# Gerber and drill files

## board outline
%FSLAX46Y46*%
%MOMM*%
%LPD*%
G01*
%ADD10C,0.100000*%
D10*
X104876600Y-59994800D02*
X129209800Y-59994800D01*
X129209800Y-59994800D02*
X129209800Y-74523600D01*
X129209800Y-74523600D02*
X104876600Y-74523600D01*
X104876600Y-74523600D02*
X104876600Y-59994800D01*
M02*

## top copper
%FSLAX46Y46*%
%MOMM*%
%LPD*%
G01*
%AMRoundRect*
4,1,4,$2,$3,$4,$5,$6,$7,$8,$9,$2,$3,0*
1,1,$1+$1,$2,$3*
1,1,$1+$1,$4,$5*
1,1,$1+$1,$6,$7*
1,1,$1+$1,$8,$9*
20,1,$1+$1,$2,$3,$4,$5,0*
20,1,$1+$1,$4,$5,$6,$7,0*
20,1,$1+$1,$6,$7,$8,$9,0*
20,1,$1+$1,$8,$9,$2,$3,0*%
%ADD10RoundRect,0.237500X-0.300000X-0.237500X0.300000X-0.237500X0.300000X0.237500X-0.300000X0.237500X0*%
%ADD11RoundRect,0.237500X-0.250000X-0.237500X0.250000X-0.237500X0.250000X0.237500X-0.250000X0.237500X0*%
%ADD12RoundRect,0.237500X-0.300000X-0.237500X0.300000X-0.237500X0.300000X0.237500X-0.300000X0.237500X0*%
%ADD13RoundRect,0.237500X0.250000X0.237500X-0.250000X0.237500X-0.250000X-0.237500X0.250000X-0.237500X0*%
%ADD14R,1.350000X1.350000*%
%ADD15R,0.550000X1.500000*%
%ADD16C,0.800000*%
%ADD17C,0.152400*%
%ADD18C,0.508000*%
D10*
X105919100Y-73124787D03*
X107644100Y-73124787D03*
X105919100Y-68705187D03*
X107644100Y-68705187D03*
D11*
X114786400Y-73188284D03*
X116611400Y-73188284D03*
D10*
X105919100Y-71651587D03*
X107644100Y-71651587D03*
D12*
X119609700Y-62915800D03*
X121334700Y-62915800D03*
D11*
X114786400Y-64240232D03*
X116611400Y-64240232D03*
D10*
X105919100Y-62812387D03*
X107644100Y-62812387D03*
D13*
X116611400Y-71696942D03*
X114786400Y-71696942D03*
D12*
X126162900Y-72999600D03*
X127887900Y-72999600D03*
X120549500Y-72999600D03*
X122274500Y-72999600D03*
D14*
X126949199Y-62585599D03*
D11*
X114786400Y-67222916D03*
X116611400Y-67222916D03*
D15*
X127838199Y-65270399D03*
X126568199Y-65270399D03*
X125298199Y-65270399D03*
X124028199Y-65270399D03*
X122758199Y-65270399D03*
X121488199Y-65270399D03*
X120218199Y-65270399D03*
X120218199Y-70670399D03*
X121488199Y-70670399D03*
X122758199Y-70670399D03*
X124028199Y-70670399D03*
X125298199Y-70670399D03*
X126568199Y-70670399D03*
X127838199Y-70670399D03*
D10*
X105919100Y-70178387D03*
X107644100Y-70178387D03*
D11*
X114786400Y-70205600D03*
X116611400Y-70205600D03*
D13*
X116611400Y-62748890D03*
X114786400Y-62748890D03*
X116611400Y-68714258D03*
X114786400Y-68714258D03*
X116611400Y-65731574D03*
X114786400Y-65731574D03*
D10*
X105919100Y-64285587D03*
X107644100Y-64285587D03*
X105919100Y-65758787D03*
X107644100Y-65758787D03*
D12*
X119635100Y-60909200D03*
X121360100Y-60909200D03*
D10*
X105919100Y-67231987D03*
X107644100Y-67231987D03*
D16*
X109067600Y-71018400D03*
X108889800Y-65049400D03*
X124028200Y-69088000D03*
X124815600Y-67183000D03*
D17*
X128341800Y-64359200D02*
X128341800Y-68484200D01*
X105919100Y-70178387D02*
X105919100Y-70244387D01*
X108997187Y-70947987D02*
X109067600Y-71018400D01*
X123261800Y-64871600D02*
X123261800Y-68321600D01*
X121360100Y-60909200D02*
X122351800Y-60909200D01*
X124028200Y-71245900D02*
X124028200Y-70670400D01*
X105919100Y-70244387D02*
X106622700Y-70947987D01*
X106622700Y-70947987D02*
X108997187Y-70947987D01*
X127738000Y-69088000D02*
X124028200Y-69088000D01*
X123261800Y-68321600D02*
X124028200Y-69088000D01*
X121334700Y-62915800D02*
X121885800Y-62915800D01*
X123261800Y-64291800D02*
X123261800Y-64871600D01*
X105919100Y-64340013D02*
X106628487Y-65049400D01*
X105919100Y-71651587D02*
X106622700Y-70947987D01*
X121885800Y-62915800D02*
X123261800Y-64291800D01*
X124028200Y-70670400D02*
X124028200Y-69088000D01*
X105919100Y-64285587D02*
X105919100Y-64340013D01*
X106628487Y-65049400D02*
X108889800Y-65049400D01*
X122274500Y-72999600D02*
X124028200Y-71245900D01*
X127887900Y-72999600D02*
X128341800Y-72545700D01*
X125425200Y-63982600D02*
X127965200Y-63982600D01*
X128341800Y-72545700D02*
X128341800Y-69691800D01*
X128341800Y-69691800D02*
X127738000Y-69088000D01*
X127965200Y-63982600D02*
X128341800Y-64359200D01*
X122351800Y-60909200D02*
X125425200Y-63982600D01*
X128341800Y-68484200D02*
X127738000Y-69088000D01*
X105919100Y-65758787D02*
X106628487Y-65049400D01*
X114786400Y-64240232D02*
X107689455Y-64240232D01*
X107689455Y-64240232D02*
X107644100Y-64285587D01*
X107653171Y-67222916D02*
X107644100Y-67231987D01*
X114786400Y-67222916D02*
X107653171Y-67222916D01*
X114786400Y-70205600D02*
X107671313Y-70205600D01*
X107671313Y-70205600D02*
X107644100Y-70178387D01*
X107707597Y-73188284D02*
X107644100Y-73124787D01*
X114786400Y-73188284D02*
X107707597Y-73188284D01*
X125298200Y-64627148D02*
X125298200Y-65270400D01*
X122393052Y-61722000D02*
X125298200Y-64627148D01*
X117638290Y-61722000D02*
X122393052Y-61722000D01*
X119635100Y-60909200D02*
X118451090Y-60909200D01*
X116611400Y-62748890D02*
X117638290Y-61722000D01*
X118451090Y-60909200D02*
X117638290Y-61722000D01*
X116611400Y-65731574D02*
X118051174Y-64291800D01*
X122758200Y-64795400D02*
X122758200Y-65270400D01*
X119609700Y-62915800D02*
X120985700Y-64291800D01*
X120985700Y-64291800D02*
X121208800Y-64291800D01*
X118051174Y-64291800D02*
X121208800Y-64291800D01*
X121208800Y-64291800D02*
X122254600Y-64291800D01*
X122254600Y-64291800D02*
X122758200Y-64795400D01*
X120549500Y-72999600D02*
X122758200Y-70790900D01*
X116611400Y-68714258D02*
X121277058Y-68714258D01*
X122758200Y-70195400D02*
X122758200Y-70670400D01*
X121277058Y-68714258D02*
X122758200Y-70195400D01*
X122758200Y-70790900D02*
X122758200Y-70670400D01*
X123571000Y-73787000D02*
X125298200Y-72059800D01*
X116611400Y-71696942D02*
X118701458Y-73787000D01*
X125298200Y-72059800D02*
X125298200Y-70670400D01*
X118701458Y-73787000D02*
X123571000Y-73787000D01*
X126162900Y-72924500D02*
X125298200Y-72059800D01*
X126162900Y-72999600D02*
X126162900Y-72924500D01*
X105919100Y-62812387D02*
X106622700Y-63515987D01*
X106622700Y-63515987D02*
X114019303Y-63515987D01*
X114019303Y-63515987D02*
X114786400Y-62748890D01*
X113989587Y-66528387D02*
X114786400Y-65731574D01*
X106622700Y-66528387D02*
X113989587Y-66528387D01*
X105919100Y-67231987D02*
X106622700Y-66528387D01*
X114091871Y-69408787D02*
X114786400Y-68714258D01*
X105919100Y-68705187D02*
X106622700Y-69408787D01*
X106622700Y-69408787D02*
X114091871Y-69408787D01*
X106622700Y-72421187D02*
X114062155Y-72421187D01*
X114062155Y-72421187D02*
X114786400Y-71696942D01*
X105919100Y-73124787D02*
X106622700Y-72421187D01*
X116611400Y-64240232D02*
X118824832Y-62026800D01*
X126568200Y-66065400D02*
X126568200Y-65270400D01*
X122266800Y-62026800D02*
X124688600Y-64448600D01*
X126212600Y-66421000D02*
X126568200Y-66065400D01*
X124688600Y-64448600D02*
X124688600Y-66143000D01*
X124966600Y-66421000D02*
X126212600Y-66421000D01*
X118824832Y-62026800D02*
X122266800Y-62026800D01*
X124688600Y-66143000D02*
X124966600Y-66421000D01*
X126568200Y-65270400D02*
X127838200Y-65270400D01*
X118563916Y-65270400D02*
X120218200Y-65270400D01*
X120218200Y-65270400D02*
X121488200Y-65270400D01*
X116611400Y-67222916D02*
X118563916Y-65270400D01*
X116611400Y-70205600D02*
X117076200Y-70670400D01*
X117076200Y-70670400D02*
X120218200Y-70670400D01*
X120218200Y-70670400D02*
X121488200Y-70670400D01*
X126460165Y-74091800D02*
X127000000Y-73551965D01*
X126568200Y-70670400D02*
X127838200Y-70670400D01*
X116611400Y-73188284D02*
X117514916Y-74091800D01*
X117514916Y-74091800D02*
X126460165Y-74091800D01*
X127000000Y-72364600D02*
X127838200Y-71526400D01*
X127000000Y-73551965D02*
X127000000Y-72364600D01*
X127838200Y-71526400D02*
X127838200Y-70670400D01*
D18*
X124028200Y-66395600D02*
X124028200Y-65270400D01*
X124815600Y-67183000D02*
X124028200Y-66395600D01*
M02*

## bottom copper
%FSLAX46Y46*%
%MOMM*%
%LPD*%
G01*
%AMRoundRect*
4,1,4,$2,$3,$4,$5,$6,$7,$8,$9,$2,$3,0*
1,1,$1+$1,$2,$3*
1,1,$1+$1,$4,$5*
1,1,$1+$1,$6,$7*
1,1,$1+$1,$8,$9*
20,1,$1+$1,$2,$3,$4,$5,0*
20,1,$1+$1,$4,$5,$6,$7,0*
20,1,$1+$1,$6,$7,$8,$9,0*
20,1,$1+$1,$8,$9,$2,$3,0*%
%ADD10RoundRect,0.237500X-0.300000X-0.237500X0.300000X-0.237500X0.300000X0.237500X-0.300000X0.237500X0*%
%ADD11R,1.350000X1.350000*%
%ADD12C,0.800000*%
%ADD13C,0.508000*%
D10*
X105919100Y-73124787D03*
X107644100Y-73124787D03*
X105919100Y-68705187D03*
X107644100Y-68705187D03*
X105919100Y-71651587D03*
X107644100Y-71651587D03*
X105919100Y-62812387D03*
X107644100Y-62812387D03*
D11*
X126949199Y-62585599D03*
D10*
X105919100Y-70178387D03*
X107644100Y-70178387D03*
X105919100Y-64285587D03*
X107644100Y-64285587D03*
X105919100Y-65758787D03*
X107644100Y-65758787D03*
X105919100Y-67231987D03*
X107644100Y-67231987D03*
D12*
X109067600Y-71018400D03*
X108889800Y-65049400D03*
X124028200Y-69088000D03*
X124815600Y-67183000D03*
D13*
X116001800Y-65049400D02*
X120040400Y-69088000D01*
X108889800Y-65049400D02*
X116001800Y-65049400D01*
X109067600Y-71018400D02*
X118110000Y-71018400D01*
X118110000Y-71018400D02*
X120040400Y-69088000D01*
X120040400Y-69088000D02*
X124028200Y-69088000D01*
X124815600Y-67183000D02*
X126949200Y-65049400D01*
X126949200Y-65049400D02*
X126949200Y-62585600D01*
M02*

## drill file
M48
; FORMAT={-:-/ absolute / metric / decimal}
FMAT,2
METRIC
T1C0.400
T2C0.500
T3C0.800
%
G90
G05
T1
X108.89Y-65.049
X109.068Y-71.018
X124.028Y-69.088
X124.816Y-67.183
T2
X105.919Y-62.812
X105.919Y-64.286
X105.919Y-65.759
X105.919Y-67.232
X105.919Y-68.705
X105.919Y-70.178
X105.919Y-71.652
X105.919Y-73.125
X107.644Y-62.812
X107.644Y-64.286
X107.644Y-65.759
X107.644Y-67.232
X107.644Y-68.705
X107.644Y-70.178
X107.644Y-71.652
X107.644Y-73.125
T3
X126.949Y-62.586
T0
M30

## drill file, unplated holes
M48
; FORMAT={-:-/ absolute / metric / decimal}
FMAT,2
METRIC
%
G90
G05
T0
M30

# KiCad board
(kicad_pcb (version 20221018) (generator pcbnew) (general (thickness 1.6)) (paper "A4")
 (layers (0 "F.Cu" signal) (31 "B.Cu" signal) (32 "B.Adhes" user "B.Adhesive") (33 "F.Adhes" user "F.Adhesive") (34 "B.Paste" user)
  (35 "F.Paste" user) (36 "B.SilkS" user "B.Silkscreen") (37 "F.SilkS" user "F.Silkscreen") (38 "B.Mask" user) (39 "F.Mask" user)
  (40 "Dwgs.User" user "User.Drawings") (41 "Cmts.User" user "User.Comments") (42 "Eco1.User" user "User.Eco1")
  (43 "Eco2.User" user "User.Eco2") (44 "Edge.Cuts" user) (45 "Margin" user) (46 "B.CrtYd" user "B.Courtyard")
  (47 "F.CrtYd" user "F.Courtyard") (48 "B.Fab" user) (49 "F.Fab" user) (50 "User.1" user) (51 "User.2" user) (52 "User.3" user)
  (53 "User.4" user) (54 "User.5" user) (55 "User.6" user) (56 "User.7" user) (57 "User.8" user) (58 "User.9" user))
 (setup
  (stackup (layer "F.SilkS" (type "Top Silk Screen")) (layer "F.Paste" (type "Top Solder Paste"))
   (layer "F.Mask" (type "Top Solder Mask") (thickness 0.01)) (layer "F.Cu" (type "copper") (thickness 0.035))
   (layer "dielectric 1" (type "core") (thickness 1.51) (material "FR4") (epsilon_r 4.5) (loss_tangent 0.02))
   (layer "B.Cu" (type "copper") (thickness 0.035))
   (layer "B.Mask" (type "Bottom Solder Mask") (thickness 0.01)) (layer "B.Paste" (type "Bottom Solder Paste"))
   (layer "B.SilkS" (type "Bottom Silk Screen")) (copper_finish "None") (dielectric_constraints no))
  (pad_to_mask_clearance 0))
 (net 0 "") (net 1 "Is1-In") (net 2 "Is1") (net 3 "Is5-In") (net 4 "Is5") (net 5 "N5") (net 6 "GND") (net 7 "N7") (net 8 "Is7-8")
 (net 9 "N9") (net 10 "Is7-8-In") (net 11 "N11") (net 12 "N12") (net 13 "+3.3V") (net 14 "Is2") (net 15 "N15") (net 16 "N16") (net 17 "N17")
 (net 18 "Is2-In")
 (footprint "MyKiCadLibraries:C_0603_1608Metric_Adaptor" (layer "F.Cu") (at 106.7816 73.124787)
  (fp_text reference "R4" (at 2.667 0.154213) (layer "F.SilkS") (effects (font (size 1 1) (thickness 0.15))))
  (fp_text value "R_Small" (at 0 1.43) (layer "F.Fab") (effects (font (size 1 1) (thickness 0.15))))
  (pad "1" thru_hole roundrect (at -0.8625 0) (size 1.075 0.95) (drill 0.5) (layers "*.Cu" "*.Mask") (roundrect_rratio 0.25)
   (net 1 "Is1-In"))
  (pad "2" thru_hole roundrect (at 0.8625 0) (size 1.075 0.95) (drill 0.5) (layers "*.Cu" "*.Mask") (roundrect_rratio 0.25) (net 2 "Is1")))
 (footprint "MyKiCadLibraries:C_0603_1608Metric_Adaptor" (layer "F.Cu") (at 106.7816 68.705187)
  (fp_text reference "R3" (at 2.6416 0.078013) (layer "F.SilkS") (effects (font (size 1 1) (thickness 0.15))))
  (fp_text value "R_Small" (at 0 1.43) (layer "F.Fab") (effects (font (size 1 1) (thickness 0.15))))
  (pad "1" thru_hole roundrect (at -0.8625 0) (size 1.075 0.95) (drill 0.5) (layers "*.Cu" "*.Mask") (roundrect_rratio 0.25)
   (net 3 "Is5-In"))
  (pad "2" thru_hole roundrect (at 0.8625 0) (size 1.075 0.95) (drill 0.5) (layers "*.Cu" "*.Mask") (roundrect_rratio 0.25) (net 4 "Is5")))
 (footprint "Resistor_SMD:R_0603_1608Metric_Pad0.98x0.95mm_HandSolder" (layer "F.Cu") (at 115.6989 73.188284)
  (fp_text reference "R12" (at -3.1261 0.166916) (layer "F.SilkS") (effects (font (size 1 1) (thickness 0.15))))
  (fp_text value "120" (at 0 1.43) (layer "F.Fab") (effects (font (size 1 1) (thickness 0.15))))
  (pad "1" smd roundrect (at -0.9125 0) (size 0.975 0.95) (layers "F.Cu" "F.Paste" "F.Mask") (roundrect_rratio 0.25) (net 2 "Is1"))
  (pad "2" smd roundrect (at 0.9125 0) (size 0.975 0.95) (layers "F.Cu" "F.Paste" "F.Mask") (roundrect_rratio 0.25) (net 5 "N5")))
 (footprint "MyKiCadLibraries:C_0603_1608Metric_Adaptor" (layer "F.Cu") (at 106.7816 71.651587)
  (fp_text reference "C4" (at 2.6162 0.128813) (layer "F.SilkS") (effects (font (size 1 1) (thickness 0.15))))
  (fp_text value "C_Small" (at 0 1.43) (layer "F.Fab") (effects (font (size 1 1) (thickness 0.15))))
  (pad "1" thru_hole roundrect (at -0.8625 0) (size 1.075 0.95) (drill 0.5) (layers "*.Cu" "*.Mask") (roundrect_rratio 0.25) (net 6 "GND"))
  (pad "2" thru_hole roundrect (at 0.8625 0) (size 1.075 0.95) (drill 0.5) (layers "*.Cu" "*.Mask") (roundrect_rratio 0.25) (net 2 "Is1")))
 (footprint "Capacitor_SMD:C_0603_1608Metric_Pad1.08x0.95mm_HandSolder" (layer "F.Cu") (at 120.4722 62.9158)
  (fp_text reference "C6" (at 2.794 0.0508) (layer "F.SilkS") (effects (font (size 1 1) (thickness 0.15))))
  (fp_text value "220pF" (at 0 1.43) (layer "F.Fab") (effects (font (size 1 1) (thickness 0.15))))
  (pad "1" smd roundrect (at -0.8625 0) (size 1.075 0.95) (layers "F.Cu" "F.Paste" "F.Mask") (roundrect_rratio 0.25) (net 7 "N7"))
  (pad "2" smd roundrect (at 0.8625 0) (size 1.075 0.95) (layers "F.Cu" "F.Paste" "F.Mask") (roundrect_rratio 0.25) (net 6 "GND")))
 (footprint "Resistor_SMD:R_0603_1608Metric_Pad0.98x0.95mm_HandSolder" (layer "F.Cu") (at 115.6989 64.240232)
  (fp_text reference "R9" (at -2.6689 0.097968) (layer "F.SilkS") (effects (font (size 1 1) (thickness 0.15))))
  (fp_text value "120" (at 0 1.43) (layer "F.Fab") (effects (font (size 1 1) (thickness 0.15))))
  (pad "1" smd roundrect (at -0.9125 0) (size 0.975 0.95) (layers "F.Cu" "F.Paste" "F.Mask") (roundrect_rratio 0.25) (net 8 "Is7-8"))
  (pad "2" smd roundrect (at 0.9125 0) (size 0.975 0.95) (layers "F.Cu" "F.Paste" "F.Mask") (roundrect_rratio 0.25) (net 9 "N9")))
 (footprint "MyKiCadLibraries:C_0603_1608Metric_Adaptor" (layer "F.Cu") (at 106.7816 62.812387)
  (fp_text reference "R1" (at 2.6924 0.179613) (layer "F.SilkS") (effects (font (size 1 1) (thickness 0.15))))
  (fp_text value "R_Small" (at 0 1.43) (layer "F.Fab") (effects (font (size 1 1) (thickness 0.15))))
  (pad "1" thru_hole roundrect (at -0.8625 0) (size 1.075 0.95) (drill 0.5) (layers "*.Cu" "*.Mask") (roundrect_rratio 0.25)
   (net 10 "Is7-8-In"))
  (pad "2" thru_hole roundrect (at 0.8625 0) (size 1.075 0.95) (drill 0.5) (layers "*.Cu" "*.Mask") (roundrect_rratio 0.25) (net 8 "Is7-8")))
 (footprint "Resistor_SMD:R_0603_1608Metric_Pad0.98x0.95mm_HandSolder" (layer "F.Cu") (at 115.6989 71.696942 180)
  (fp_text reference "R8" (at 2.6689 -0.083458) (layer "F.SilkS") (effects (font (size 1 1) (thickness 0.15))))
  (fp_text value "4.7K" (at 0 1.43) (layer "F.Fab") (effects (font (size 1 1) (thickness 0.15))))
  (pad "1" smd roundrect (at -0.9125 0 180) (size 0.975 0.95) (layers "F.Cu" "F.Paste" "F.Mask") (roundrect_rratio 0.25) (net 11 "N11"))
  (pad "2" smd roundrect (at 0.9125 0 180) (size 0.975 0.95) (layers "F.Cu" "F.Paste" "F.Mask") (roundrect_rratio 0.25) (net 1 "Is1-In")))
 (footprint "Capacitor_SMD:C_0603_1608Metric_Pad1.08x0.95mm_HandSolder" (layer "F.Cu") (at 127.0254 72.9996)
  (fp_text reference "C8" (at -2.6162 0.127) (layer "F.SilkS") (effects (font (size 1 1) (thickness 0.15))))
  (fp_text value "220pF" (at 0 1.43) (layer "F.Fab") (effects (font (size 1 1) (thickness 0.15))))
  (pad "1" smd roundrect (at -0.8625 0) (size 1.075 0.95) (layers "F.Cu" "F.Paste" "F.Mask") (roundrect_rratio 0.25) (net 11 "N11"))
  (pad "2" smd roundrect (at 0.8625 0) (size 1.075 0.95) (layers "F.Cu" "F.Paste" "F.Mask") (roundrect_rratio 0.25) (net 6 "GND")))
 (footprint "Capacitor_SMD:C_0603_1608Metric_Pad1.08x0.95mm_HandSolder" (layer "F.Cu") (at 121.412 72.9996)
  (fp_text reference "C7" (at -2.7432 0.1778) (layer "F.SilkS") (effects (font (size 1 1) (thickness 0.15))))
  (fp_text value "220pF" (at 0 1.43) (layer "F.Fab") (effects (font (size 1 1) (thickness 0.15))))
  (pad "1" smd roundrect (at -0.8625 0) (size 1.075 0.95) (layers "F.Cu" "F.Paste" "F.Mask") (roundrect_rratio 0.25) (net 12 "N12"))
  (pad "2" smd roundrect (at 0.8625 0) (size 1.075 0.95) (layers "F.Cu" "F.Paste" "F.Mask") (roundrect_rratio 0.25) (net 6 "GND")))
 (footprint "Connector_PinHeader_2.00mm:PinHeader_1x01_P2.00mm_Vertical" (layer "F.Cu") (at 126.9492 62.5856)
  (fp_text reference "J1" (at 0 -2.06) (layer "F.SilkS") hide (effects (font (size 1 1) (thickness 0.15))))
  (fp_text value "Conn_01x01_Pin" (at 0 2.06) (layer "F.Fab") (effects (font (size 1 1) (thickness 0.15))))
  (pad "1" thru_hole rect (at 0 0) (size 1.35 1.35) (drill 0.8) (layers "*.Cu" "*.Mask") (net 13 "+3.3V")))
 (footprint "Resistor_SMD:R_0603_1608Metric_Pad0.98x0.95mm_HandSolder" (layer "F.Cu") (at 115.6989 67.222916)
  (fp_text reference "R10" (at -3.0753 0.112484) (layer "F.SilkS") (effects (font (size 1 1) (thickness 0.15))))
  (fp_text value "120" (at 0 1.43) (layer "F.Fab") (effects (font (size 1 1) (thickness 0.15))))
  (pad "1" smd roundrect (at -0.9125 0) (size 0.975 0.95) (layers "F.Cu" "F.Paste" "F.Mask") (roundrect_rratio 0.25) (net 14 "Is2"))
  (pad "2" smd roundrect (at 0.9125 0) (size 0.975 0.95) (layers "F.Cu" "F.Paste" "F.Mask") (roundrect_rratio 0.25) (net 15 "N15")))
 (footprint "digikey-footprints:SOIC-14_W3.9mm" (layer "F.Cu") (at 124.0282 67.9704 180)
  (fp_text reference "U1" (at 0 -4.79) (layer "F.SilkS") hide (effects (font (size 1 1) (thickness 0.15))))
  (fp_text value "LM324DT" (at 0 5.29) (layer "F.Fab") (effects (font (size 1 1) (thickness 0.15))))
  (pad "1" smd rect (at -3.81 2.7 180) (size 0.55 1.5) (layers "F.Cu" "F.Paste" "F.Mask") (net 9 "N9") (solder_mask_margin 0.07))
  (pad "2" smd rect (at -2.54 2.7 180) (size 0.55 1.5) (layers "F.Cu" "F.Paste" "F.Mask") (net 9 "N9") (solder_mask_margin 0.07))
  (pad "3" smd rect (at -1.27 2.7 180) (size 0.55 1.5) (layers "F.Cu" "F.Paste" "F.Mask") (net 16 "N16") (solder_mask_margin 0.07))
  (pad "4" smd rect (at 0 2.7 180) (size 0.55 1.5) (layers "F.Cu" "F.Paste" "F.Mask") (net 13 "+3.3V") (solder_mask_margin 0.07))
  (pad "5" smd rect (at 1.27 2.7 180) (size 0.55 1.5) (layers "F.Cu" "F.Paste" "F.Mask") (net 7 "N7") (solder_mask_margin 0.07))
  (pad "6" smd rect (at 2.54 2.7 180) (size 0.55 1.5) (layers "F.Cu" "F.Paste" "F.Mask") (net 15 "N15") (solder_mask_margin 0.07))
  (pad "7" smd rect (at 3.81 2.7 180) (size 0.55 1.5) (layers "F.Cu" "F.Paste" "F.Mask") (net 15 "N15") (solder_mask_margin 0.07))
  (pad "8" smd rect (at 3.81 -2.7 180) (size 0.55 1.5) (layers "F.Cu" "F.Paste" "F.Mask") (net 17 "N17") (solder_mask_margin 0.07))
  (pad "9" smd rect (at 2.54 -2.7 180) (size 0.55 1.5) (layers "F.Cu" "F.Paste" "F.Mask") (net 17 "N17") (solder_mask_margin 0.07))
  (pad "10" smd rect (at 1.27 -2.7 180) (size 0.55 1.5) (layers "F.Cu" "F.Paste" "F.Mask") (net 12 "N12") (solder_mask_margin 0.07))
  (pad "11" smd rect (at 0 -2.7 180) (size 0.55 1.5) (layers "F.Cu" "F.Paste" "F.Mask") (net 6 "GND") (solder_mask_margin 0.07))
  (pad "12" smd rect (at -1.27 -2.7 180) (size 0.55 1.5) (layers "F.Cu" "F.Paste" "F.Mask") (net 11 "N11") (solder_mask_margin 0.07))
  (pad "13" smd rect (at -2.54 -2.7 180) (size 0.55 1.5) (layers "F.Cu" "F.Paste" "F.Mask") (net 5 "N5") (solder_mask_margin 0.07))
  (pad "14" smd rect (at -3.81 -2.7 180) (size 0.55 1.5) (layers "F.Cu" "F.Paste" "F.Mask") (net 5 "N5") (solder_mask_margin 0.07)))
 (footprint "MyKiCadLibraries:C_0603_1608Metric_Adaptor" (layer "F.Cu") (at 106.7816 70.178387)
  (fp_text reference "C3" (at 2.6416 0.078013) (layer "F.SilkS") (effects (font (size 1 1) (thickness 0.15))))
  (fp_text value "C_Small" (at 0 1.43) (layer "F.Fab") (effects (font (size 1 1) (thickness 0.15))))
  (pad "1" thru_hole roundrect (at -0.8625 0) (size 1.075 0.95) (drill 0.5) (layers "*.Cu" "*.Mask") (roundrect_rratio 0.25) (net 6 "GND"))
  (pad "2" thru_hole roundrect (at 0.8625 0) (size 1.075 0.95) (drill 0.5) (layers "*.Cu" "*.Mask") (roundrect_rratio 0.25) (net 4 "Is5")))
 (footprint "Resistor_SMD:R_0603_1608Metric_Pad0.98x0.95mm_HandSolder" (layer "F.Cu") (at 115.6989 70.2056)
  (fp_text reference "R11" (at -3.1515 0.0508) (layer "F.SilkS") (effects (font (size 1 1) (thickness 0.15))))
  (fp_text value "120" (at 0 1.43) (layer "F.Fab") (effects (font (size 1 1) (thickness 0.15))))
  (pad "1" smd roundrect (at -0.9125 0) (size 0.975 0.95) (layers "F.Cu" "F.Paste" "F.Mask") (roundrect_rratio 0.25) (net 4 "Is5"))
  (pad "2" smd roundrect (at 0.9125 0) (size 0.975 0.95) (layers "F.Cu" "F.Paste" "F.Mask") (roundrect_rratio 0.25) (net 17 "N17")))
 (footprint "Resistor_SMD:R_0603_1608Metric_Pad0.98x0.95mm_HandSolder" (layer "F.Cu") (at 115.6989 62.74889 180)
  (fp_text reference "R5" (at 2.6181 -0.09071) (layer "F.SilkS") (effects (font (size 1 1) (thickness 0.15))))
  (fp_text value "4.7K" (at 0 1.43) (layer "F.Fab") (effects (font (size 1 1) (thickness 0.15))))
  (pad "1" smd roundrect (at -0.9125 0 180) (size 0.975 0.95) (layers "F.Cu" "F.Paste" "F.Mask") (roundrect_rratio 0.25) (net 16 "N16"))
  (pad "2" smd roundrect (at 0.9125 0 180) (size 0.975 0.95) (layers "F.Cu" "F.Paste" "F.Mask") (roundrect_rratio 0.25) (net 10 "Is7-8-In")))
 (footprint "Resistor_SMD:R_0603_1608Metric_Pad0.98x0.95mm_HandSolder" (layer "F.Cu") (at 115.6989 68.714258 180)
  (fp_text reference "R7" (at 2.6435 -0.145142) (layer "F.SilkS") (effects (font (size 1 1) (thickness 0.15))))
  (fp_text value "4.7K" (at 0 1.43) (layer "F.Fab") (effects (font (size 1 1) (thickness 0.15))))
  (pad "1" smd roundrect (at -0.9125 0 180) (size 0.975 0.95) (layers "F.Cu" "F.Paste" "F.Mask") (roundrect_rratio 0.25) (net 12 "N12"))
  (pad "2" smd roundrect (at 0.9125 0 180) (size 0.975 0.95) (layers "F.Cu" "F.Paste" "F.Mask") (roundrect_rratio 0.25) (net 3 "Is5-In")))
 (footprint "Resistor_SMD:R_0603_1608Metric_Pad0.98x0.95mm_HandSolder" (layer "F.Cu") (at 115.6989 65.731574 180)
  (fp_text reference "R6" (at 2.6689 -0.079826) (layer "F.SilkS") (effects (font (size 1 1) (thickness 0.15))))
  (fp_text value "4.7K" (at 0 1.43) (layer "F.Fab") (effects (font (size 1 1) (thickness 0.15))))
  (pad "1" smd roundrect (at -0.9125 0 180) (size 0.975 0.95) (layers "F.Cu" "F.Paste" "F.Mask") (roundrect_rratio 0.25) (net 7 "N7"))
  (pad "2" smd roundrect (at 0.9125 0 180) (size 0.975 0.95) (layers "F.Cu" "F.Paste" "F.Mask") (roundrect_rratio 0.25) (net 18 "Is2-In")))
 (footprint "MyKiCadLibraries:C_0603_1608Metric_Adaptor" (layer "F.Cu") (at 106.7816 64.285587)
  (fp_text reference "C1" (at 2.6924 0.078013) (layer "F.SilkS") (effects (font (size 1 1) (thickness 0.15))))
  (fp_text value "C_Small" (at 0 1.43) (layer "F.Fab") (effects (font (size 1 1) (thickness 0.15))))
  (pad "1" thru_hole roundrect (at -0.8625 0) (size 1.075 0.95) (drill 0.5) (layers "*.Cu" "*.Mask") (roundrect_rratio 0.25) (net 6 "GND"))
  (pad "2" thru_hole roundrect (at 0.8625 0) (size 1.075 0.95) (drill 0.5) (layers "*.Cu" "*.Mask") (roundrect_rratio 0.25) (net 8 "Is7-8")))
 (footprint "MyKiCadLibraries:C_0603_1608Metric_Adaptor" (layer "F.Cu") (at 106.7816 65.758787)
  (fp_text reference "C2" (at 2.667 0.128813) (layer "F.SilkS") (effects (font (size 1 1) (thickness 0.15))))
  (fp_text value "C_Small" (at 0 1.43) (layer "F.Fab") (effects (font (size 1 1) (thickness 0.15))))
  (pad "1" thru_hole roundrect (at -0.8625 0) (size 1.075 0.95) (drill 0.5) (layers "*.Cu" "*.Mask") (roundrect_rratio 0.25) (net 6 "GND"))
  (pad "2" thru_hole roundrect (at 0.8625 0) (size 1.075 0.95) (drill 0.5) (layers "*.Cu" "*.Mask") (roundrect_rratio 0.25) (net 14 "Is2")))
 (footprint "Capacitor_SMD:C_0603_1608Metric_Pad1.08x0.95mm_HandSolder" (layer "F.Cu") (at 120.4976 60.9092)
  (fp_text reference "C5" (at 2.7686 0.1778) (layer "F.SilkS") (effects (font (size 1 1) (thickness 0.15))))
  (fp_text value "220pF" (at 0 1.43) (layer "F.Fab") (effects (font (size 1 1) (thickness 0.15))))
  (pad "1" smd roundrect (at -0.8625 0) (size 1.075 0.95) (layers "F.Cu" "F.Paste" "F.Mask") (roundrect_rratio 0.25) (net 16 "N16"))
  (pad "2" smd roundrect (at 0.8625 0) (size 1.075 0.95) (layers "F.Cu" "F.Paste" "F.Mask") (roundrect_rratio 0.25) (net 6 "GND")))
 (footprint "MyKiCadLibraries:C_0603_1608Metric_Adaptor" (layer "F.Cu") (at 106.7816 67.231987)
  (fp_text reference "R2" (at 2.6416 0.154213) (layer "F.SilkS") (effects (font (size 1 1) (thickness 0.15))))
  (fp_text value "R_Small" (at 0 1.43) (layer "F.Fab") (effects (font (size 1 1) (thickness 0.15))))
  (pad "1" thru_hole roundrect (at -0.8625 0) (size 1.075 0.95) (drill 0.5) (layers "*.Cu" "*.Mask") (roundrect_rratio 0.25)
   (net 18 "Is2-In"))
  (pad "2" thru_hole roundrect (at 0.8625 0) (size 1.075 0.95) (drill 0.5) (layers "*.Cu" "*.Mask") (roundrect_rratio 0.25) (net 14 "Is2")))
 (gr_rect (start 104.8766 59.9948) (end 129.2098 74.5236) (stroke (width 0.1) (type default)) (fill none) (layer "Edge.Cuts"))
 (segment (start 128.3418 64.3592) (end 128.3418 68.4842) (width 0.1524) (layer "F.Cu") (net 6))
 (segment (start 105.9191 70.178387) (end 105.9191 70.244387) (width 0.1524) (layer "F.Cu") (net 6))
 (segment (start 108.997187 70.947987) (end 109.0676 71.0184) (width 0.1524) (layer "F.Cu") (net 6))
 (segment (start 123.2618 64.8716) (end 123.2618 68.3216) (width 0.1524) (layer "F.Cu") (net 6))
 (segment (start 121.3601 60.9092) (end 122.3518 60.9092) (width 0.1524) (layer "F.Cu") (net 6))
 (segment (start 124.0282 71.2459) (end 124.0282 70.6704) (width 0.1524) (layer "F.Cu") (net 6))
 (segment (start 105.9191 70.244387) (end 106.6227 70.947987) (width 0.1524) (layer "F.Cu") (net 6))
 (segment (start 106.6227 70.947987) (end 108.997187 70.947987) (width 0.1524) (layer "F.Cu") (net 6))
 (segment (start 127.738 69.088) (end 124.0282 69.088) (width 0.1524) (layer "F.Cu") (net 6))
 (segment (start 123.2618 68.3216) (end 124.0282 69.088) (width 0.1524) (layer "F.Cu") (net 6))
 (segment (start 121.3347 62.9158) (end 121.8858 62.9158) (width 0.1524) (layer "F.Cu") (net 6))
 (segment (start 123.2618 64.2918) (end 123.2618 64.8716) (width 0.1524) (layer "F.Cu") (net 6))
 (segment (start 105.9191 64.340013) (end 106.628487 65.0494) (width 0.1524) (layer "F.Cu") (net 6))
 (segment (start 105.9191 71.651587) (end 106.6227 70.947987) (width 0.1524) (layer "F.Cu") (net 6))
 (segment (start 121.8858 62.9158) (end 123.2618 64.2918) (width 0.1524) (layer "F.Cu") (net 6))
 (segment (start 124.0282 70.6704) (end 124.0282 69.088) (width 0.1524) (layer "F.Cu") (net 6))
 (segment (start 105.9191 64.285587) (end 105.9191 64.340013) (width 0.1524) (layer "F.Cu") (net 6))
 (segment (start 106.628487 65.0494) (end 108.8898 65.0494) (width 0.1524) (layer "F.Cu") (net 6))
 (segment (start 122.2745 72.9996) (end 124.0282 71.2459) (width 0.1524) (layer "F.Cu") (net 6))
 (segment (start 127.8879 72.9996) (end 128.3418 72.5457) (width 0.1524) (layer "F.Cu") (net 6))
 (segment (start 125.4252 63.9826) (end 127.9652 63.9826) (width 0.1524) (layer "F.Cu") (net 6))
 (segment (start 128.3418 72.5457) (end 128.3418 69.6918) (width 0.1524) (layer "F.Cu") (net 6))
 (segment (start 128.3418 69.6918) (end 127.738 69.088) (width 0.1524) (layer "F.Cu") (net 6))
 (segment (start 127.9652 63.9826) (end 128.3418 64.3592) (width 0.1524) (layer "F.Cu") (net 6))
 (segment (start 122.3518 60.9092) (end 125.4252 63.9826) (width 0.1524) (layer "F.Cu") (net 6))
 (segment (start 128.3418 68.4842) (end 127.738 69.088) (width 0.1524) (layer "F.Cu") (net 6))
 (segment (start 105.9191 65.758787) (end 106.628487 65.0494) (width 0.1524) (layer "F.Cu") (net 6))
 (via (at 109.0676 71.0184) (size 0.8) (drill 0.4) (layers "F.Cu" "B.Cu") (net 6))
 (via (at 108.8898 65.0494) (size 0.8) (drill 0.4) (layers "F.Cu" "B.Cu") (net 6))
 (via (at 124.0282 69.088) (size 0.8) (drill 0.4) (layers "F.Cu" "B.Cu") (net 6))
 (segment (start 116.0018 65.0494) (end 120.0404 69.088) (width 0.508) (layer "B.Cu") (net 6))
 (segment (start 108.8898 65.0494) (end 116.0018 65.0494) (width 0.508) (layer "B.Cu") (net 6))
 (segment (start 109.0676 71.0184) (end 118.11 71.0184) (width 0.508) (layer "B.Cu") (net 6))
 (segment (start 118.11 71.0184) (end 120.0404 69.088) (width 0.508) (layer "B.Cu") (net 6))
 (segment (start 120.0404 69.088) (end 124.0282 69.088) (width 0.508) (layer "B.Cu") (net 6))
 (segment (start 114.7864 64.240232) (end 107.689455 64.240232) (width 0.1524) (layer "F.Cu") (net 8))
 (segment (start 107.689455 64.240232) (end 107.6441 64.285587) (width 0.1524) (layer "F.Cu") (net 8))
 (segment (start 107.653171 67.222916) (end 107.6441 67.231987) (width 0.1524) (layer "F.Cu") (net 14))
 (segment (start 114.7864 67.222916) (end 107.653171 67.222916) (width 0.1524) (layer "F.Cu") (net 14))
 (segment (start 114.7864 70.2056) (end 107.671313 70.2056) (width 0.1524) (layer "F.Cu") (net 4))
 (segment (start 107.671313 70.2056) (end 107.6441 70.178387) (width 0.1524) (layer "F.Cu") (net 4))
 (segment (start 107.707597 73.188284) (end 107.6441 73.124787) (width 0.1524) (layer "F.Cu") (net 2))
 (segment (start 114.7864 73.188284) (end 107.707597 73.188284) (width 0.1524) (layer "F.Cu") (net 2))
 (segment (start 125.2982 64.627148) (end 125.2982 65.2704) (width 0.1524) (layer "F.Cu") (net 16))
 (segment (start 122.393052 61.722) (end 125.2982 64.627148) (width 0.1524) (layer "F.Cu") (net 16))
 (segment (start 117.63829 61.722) (end 122.393052 61.722) (width 0.1524) (layer "F.Cu") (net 16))
 (segment (start 119.6351 60.9092) (end 118.45109 60.9092) (width 0.1524) (layer "F.Cu") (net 16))
 (segment (start 116.6114 62.74889) (end 117.63829 61.722) (width 0.1524) (layer "F.Cu") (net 16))
 (segment (start 118.45109 60.9092) (end 117.63829 61.722) (width 0.1524) (layer "F.Cu") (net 16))
 (segment (start 116.6114 65.731574) (end 118.051174 64.2918) (width 0.1524) (layer "F.Cu") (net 7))
 (segment (start 122.7582 64.7954) (end 122.7582 65.2704) (width 0.1524) (layer "F.Cu") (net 7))
 (segment (start 119.6097 62.9158) (end 120.9857 64.2918) (width 0.1524) (layer "F.Cu") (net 7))
 (segment (start 120.9857 64.2918) (end 121.2088 64.2918) (width 0.1524) (layer "F.Cu") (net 7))
 (segment (start 118.051174 64.2918) (end 121.2088 64.2918) (width 0.1524) (layer "F.Cu") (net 7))
 (segment (start 121.2088 64.2918) (end 122.2546 64.2918) (width 0.1524) (layer "F.Cu") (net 7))
 (segment (start 122.2546 64.2918) (end 122.7582 64.7954) (width 0.1524) (layer "F.Cu") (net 7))
 (segment (start 120.5495 72.9996) (end 122.7582 70.7909) (width 0.1524) (layer "F.Cu") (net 12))
 (segment (start 116.6114 68.714258) (end 121.277058 68.714258) (width 0.1524) (layer "F.Cu") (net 12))
 (segment (start 122.7582 70.1954) (end 122.7582 70.6704) (width 0.1524) (layer "F.Cu") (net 12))
 (segment (start 121.277058 68.714258) (end 122.7582 70.1954) (width 0.1524) (layer "F.Cu") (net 12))
 (segment (start 122.7582 70.7909) (end 122.7582 70.6704) (width 0.1524) (layer "F.Cu") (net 12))
 (segment (start 123.571 73.787) (end 125.2982 72.0598) (width 0.1524) (layer "F.Cu") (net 11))
 (segment (start 116.6114 71.696942) (end 118.701458 73.787) (width 0.1524) (layer "F.Cu") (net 11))
 (segment (start 125.2982 72.0598) (end 125.2982 70.6704) (width 0.1524) (layer "F.Cu") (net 11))
 (segment (start 118.701458 73.787) (end 123.571 73.787) (width 0.1524) (layer "F.Cu") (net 11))
 (segment (start 126.1629 72.9245) (end 125.2982 72.0598) (width 0.1524) (layer "F.Cu") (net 11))
 (segment (start 126.1629 72.9996) (end 126.1629 72.9245) (width 0.1524) (layer "F.Cu") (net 11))
 (segment (start 105.9191 62.812387) (end 106.6227 63.515987) (width 0.1524) (layer "F.Cu") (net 10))
 (segment (start 106.6227 63.515987) (end 114.019303 63.515987) (width 0.1524) (layer "F.Cu") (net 10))
 (segment (start 114.019303 63.515987) (end 114.7864 62.74889) (width 0.1524) (layer "F.Cu") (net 10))
 (segment (start 113.989587 66.528387) (end 114.7864 65.731574) (width 0.1524) (layer "F.Cu") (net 18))
 (segment (start 106.6227 66.528387) (end 113.989587 66.528387) (width 0.1524) (layer "F.Cu") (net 18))
 (segment (start 105.9191 67.231987) (end 106.6227 66.528387) (width 0.1524) (layer "F.Cu") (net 18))
 (segment (start 114.091871 69.408787) (end 114.7864 68.714258) (width 0.1524) (layer "F.Cu") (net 3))
 (segment (start 105.9191 68.705187) (end 106.6227 69.408787) (width 0.1524) (layer "F.Cu") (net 3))
 (segment (start 106.6227 69.408787) (end 114.091871 69.408787) (width 0.1524) (layer "F.Cu") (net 3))
 (segment (start 106.6227 72.421187) (end 114.062155 72.421187) (width 0.1524) (layer "F.Cu") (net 1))
 (segment (start 114.062155 72.421187) (end 114.7864 71.696942) (width 0.1524) (layer "F.Cu") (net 1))
 (segment (start 105.9191 73.124787) (end 106.6227 72.421187) (width 0.1524) (layer "F.Cu") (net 1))
 (segment (start 116.6114 64.240232) (end 118.824832 62.0268) (width 0.1524) (layer "F.Cu") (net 9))
 (segment (start 126.5682 66.0654) (end 126.5682 65.2704) (width 0.1524) (layer "F.Cu") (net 9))
 (segment (start 122.2668 62.0268) (end 124.6886 64.4486) (width 0.1524) (layer "F.Cu") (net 9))
 (segment (start 126.2126 66.421) (end 126.5682 66.0654) (width 0.1524) (layer "F.Cu") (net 9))
 (segment (start 124.6886 64.4486) (end 124.6886 66.143) (width 0.1524) (layer "F.Cu") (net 9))
 (segment (start 124.9666 66.421) (end 126.2126 66.421) (width 0.1524) (layer "F.Cu") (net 9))
 (segment (start 118.824832 62.0268) (end 122.2668 62.0268) (width 0.1524) (layer "F.Cu") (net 9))
 (segment (start 124.6886 66.143) (end 124.9666 66.421) (width 0.1524) (layer "F.Cu") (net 9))
 (segment (start 126.5682 65.2704) (end 127.8382 65.2704) (width 0.1524) (layer "F.Cu") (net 9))
 (segment (start 118.563916 65.2704) (end 120.2182 65.2704) (width 0.1524) (layer "F.Cu") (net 15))
 (segment (start 120.2182 65.2704) (end 121.4882 65.2704) (width 0.1524) (layer "F.Cu") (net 15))
 (segment (start 116.6114 67.222916) (end 118.563916 65.2704) (width 0.1524) (layer "F.Cu") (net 15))
 (segment (start 116.6114 70.2056) (end 117.0762 70.6704) (width 0.1524) (layer "F.Cu") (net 17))
 (segment (start 117.0762 70.6704) (end 120.2182 70.6704) (width 0.1524) (layer "F.Cu") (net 17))
 (segment (start 120.2182 70.6704) (end 121.4882 70.6704) (width 0.1524) (layer "F.Cu") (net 17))
 (segment (start 126.460165 74.0918) (end 127 73.551965) (width 0.1524) (layer "F.Cu") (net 5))
 (segment (start 126.5682 70.6704) (end 127.8382 70.6704) (width 0.1524) (layer "F.Cu") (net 5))
 (segment (start 116.6114 73.188284) (end 117.514916 74.0918) (width 0.1524) (layer "F.Cu") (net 5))
 (segment (start 117.514916 74.0918) (end 126.460165 74.0918) (width 0.1524) (layer "F.Cu") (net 5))
 (segment (start 127 72.3646) (end 127.8382 71.5264) (width 0.1524) (layer "F.Cu") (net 5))
 (segment (start 127 73.551965) (end 127 72.3646) (width 0.1524) (layer "F.Cu") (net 5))
 (segment (start 127.8382 71.5264) (end 127.8382 70.6704) (width 0.1524) (layer "F.Cu") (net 5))
 (segment (start 124.0282 66.3956) (end 124.0282 65.2704) (width 0.508) (layer "F.Cu") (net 13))
 (segment (start 124.8156 67.183) (end 124.0282 66.3956) (width 0.508) (layer "F.Cu") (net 13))
 (via (at 124.8156 67.183) (size 0.8) (drill 0.4) (layers "F.Cu" "B.Cu") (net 13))
 (segment (start 124.8156 67.183) (end 126.9492 65.0494) (width 0.508) (layer "B.Cu") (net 13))
 (segment (start 126.9492 65.0494) (end 126.9492 62.5856) (width 0.508) (layer "B.Cu") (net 13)))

